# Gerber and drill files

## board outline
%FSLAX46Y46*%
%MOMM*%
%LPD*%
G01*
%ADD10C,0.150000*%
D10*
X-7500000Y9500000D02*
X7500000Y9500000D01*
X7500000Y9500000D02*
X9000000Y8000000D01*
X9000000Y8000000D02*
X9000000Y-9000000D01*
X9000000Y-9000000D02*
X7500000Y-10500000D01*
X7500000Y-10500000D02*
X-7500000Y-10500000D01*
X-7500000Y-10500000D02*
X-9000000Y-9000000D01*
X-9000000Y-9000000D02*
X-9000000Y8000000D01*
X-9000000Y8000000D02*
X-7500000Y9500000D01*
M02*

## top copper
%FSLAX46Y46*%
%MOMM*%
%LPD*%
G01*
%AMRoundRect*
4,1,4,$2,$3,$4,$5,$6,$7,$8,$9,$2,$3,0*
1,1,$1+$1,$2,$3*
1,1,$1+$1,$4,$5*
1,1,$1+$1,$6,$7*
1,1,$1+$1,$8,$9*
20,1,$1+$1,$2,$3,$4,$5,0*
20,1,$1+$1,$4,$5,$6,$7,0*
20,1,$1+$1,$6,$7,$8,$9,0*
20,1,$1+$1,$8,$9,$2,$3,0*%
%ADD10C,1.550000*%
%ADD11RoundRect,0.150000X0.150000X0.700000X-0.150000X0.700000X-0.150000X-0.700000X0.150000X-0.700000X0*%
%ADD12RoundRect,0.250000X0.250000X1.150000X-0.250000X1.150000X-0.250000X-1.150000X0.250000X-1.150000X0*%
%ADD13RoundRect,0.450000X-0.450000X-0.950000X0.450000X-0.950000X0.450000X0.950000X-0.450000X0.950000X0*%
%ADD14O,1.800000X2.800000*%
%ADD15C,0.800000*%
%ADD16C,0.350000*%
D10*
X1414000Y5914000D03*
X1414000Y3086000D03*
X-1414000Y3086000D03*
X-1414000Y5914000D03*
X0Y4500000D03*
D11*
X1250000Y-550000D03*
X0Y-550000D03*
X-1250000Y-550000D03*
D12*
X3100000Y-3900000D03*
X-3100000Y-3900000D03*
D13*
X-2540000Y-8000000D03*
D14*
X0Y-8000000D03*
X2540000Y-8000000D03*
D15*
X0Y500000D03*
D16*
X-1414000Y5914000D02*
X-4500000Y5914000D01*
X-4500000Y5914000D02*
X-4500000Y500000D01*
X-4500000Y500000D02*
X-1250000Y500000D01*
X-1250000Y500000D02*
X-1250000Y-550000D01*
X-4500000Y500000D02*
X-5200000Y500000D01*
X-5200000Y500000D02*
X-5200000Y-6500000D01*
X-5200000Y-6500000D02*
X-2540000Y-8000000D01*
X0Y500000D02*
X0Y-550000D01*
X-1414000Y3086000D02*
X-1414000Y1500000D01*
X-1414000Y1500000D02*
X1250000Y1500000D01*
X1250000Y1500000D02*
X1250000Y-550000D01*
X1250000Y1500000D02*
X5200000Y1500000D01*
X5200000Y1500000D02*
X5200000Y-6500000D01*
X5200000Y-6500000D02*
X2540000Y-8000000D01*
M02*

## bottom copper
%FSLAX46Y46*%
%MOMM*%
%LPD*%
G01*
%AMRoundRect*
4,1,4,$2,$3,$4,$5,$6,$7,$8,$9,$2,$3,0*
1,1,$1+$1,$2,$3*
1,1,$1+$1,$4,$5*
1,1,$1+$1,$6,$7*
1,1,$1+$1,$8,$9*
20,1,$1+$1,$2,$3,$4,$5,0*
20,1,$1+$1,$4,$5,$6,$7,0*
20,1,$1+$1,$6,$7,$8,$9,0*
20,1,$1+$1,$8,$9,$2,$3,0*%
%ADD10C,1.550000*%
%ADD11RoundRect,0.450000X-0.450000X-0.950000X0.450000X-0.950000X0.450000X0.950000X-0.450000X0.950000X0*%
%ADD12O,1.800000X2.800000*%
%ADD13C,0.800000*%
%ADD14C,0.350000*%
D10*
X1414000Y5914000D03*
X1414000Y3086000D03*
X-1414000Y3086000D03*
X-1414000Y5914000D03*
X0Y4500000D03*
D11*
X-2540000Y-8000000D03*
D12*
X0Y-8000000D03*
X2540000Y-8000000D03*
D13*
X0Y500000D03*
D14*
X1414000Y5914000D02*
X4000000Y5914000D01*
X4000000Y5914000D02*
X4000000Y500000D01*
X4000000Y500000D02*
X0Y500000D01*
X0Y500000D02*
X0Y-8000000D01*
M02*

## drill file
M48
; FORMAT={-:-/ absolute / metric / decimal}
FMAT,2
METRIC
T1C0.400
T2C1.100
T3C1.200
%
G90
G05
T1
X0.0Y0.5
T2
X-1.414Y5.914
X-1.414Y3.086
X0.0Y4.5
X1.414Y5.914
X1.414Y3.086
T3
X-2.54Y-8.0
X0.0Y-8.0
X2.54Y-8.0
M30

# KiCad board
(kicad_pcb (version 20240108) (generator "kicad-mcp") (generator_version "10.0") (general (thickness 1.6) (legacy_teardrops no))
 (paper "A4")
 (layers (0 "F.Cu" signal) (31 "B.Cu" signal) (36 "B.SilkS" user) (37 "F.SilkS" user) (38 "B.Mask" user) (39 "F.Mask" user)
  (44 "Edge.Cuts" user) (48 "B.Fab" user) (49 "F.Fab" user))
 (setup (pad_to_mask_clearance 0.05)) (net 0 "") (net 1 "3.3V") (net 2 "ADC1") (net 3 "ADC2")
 (gr_line (start -7.5 -9.5) (end 7.5 -9.5) (stroke (width 0.15) (type solid)) (layer "Edge.Cuts"))
 (gr_line (start 7.5 -9.5) (end 9.0 -8.0) (stroke (width 0.15) (type solid)) (layer "Edge.Cuts"))
 (gr_line (start 9.0 -8.0) (end 9.0 9.0) (stroke (width 0.15) (type solid)) (layer "Edge.Cuts"))
 (gr_line (start 9.0 9.0) (end 7.5 10.5) (stroke (width 0.15) (type solid)) (layer "Edge.Cuts"))
 (gr_line (start 7.5 10.5) (end -7.5 10.5) (stroke (width 0.15) (type solid)) (layer "Edge.Cuts"))
 (gr_line (start -7.5 10.5) (end -9.0 9.0) (stroke (width 0.15) (type solid)) (layer "Edge.Cuts"))
 (gr_line (start -9.0 9.0) (end -9.0 -8.0) (stroke (width 0.15) (type solid)) (layer "Edge.Cuts"))
 (gr_line (start -9.0 -8.0) (end -7.5 -9.5) (stroke (width 0.15) (type solid)) (layer "Edge.Cuts"))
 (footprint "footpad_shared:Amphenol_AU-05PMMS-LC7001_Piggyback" (layer "F.Cu") (at 0 -4.5 0)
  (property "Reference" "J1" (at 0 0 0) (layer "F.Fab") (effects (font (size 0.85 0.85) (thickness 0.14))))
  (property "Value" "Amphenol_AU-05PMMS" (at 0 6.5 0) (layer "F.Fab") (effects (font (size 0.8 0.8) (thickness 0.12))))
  (pad "1" thru_hole circle (at 1.414 -1.414) (size 1.55 1.55) (drill 1.1) (layers "*.Cu" "*.Mask") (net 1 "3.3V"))
  (pad "2" thru_hole circle (at 1.414 1.414) (size 1.55 1.55) (drill 1.1) (layers "*.Cu" "*.Mask") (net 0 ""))
  (pad "3" thru_hole circle (at -1.414 1.414) (size 1.55 1.55) (drill 1.1) (layers "*.Cu" "*.Mask") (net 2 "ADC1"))
  (pad "4" thru_hole circle (at -1.414 -1.414) (size 1.55 1.55) (drill 1.1) (layers "*.Cu" "*.Mask") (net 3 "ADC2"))
  (pad "5" thru_hole circle (at 0 0) (size 1.55 1.55) (drill 1.1) (layers "*.Cu" "*.Mask") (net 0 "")))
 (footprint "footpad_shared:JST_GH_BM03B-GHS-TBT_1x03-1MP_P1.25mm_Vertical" (layer "F.Cu") (at 0 2.5 180)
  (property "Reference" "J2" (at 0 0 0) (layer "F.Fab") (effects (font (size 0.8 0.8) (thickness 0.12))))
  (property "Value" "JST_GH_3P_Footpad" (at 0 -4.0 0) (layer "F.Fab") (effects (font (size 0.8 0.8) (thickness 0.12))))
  (pad "1" smd roundrect (at -1.25 1.95 180) (size 0.6 1.7) (layers "F.Cu" "F.Mask" "F.Paste") (roundrect_rratio 0.25) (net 2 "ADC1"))
  (pad "2" smd roundrect (at 0 1.95 180) (size 0.6 1.7) (layers "F.Cu" "F.Mask" "F.Paste") (roundrect_rratio 0.25) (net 1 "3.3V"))
  (pad "3" smd roundrect (at 1.25 1.95 180) (size 0.6 1.7) (layers "F.Cu" "F.Mask" "F.Paste") (roundrect_rratio 0.25) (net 3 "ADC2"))
  (pad "MP" smd roundrect (at -3.1 -1.4 180) (size 1 2.8) (layers "F.Cu" "F.Mask" "F.Paste") (roundrect_rratio 0.25) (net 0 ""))
  (pad "MP" smd roundrect (at 3.1 -1.4 180) (size 1 2.8) (layers "F.Cu" "F.Mask" "F.Paste") (roundrect_rratio 0.25) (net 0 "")))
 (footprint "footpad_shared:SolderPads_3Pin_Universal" (layer "F.Cu") (at 0 8.0 0)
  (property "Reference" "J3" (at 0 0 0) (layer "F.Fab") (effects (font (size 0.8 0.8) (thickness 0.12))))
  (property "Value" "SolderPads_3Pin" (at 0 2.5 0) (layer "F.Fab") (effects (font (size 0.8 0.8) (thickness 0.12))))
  (pad "1" thru_hole roundrect (at -2.54 0) (size 1.8 2.8) (drill 1.2) (layers "*.Cu" "*.Mask") (roundrect_rratio 0.25) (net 3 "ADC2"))
  (pad "2" thru_hole oval (at 0 0) (size 1.8 2.8) (drill 1.2) (layers "*.Cu" "*.Mask") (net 1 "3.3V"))
  (pad "3" thru_hole oval (at 2.54 0) (size 1.8 2.8) (drill 1.2) (layers "*.Cu" "*.Mask") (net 2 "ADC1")))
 (segment (start -1.414 -5.914) (end -4.5 -5.914) (width 0.35) (layer "F.Cu") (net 3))
 (segment (start -4.5 -5.914) (end -4.5 -0.5) (width 0.35) (layer "F.Cu") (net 3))
 (segment (start -4.5 -0.5) (end -1.25 -0.5) (width 0.35) (layer "F.Cu") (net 3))
 (segment (start -1.25 -0.5) (end -1.25 0.55) (width 0.35) (layer "F.Cu") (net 3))
 (segment (start -4.5 -0.5) (end -5.2 -0.5) (width 0.35) (layer "F.Cu") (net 3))
 (segment (start -5.2 -0.5) (end -5.2 6.5) (width 0.35) (layer "F.Cu") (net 3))
 (segment (start -5.2 6.5) (end -2.54 8.0) (width 0.35) (layer "F.Cu") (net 3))
 (segment (start 1.414 -5.914) (end 4.0 -5.914) (width 0.35) (layer "B.Cu") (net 1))
 (segment (start 4.0 -5.914) (end 4.0 -0.5) (width 0.35) (layer "B.Cu") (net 1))
 (segment (start 4.0 -0.5) (end 0.0 -0.5) (width 0.35) (layer "B.Cu") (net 1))
 (via (at 0.0 -0.5) (size 0.8) (drill 0.4) (layers "F.Cu" "B.Cu") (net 1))
 (segment (start 0.0 -0.5) (end 0.0 0.55) (width 0.35) (layer "F.Cu") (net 1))
 (segment (start 0.0 -0.5) (end 0.0 8.0) (width 0.35) (layer "B.Cu") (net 1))
 (segment (start -1.414 -3.086) (end -1.414 -1.5) (width 0.35) (layer "F.Cu") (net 2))
 (segment (start -1.414 -1.5) (end 1.25 -1.5) (width 0.35) (layer "F.Cu") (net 2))
 (segment (start 1.25 -1.5) (end 1.25 0.55) (width 0.35) (layer "F.Cu") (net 2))
 (segment (start 1.25 -1.5) (end 5.2 -1.5) (width 0.35) (layer "F.Cu") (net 2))
 (segment (start 5.2 -1.5) (end 5.2 6.5) (width 0.35) (layer "F.Cu") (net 2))
 (segment (start 5.2 6.5) (end 2.54 8.0) (width 0.35) (layer "F.Cu") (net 2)))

